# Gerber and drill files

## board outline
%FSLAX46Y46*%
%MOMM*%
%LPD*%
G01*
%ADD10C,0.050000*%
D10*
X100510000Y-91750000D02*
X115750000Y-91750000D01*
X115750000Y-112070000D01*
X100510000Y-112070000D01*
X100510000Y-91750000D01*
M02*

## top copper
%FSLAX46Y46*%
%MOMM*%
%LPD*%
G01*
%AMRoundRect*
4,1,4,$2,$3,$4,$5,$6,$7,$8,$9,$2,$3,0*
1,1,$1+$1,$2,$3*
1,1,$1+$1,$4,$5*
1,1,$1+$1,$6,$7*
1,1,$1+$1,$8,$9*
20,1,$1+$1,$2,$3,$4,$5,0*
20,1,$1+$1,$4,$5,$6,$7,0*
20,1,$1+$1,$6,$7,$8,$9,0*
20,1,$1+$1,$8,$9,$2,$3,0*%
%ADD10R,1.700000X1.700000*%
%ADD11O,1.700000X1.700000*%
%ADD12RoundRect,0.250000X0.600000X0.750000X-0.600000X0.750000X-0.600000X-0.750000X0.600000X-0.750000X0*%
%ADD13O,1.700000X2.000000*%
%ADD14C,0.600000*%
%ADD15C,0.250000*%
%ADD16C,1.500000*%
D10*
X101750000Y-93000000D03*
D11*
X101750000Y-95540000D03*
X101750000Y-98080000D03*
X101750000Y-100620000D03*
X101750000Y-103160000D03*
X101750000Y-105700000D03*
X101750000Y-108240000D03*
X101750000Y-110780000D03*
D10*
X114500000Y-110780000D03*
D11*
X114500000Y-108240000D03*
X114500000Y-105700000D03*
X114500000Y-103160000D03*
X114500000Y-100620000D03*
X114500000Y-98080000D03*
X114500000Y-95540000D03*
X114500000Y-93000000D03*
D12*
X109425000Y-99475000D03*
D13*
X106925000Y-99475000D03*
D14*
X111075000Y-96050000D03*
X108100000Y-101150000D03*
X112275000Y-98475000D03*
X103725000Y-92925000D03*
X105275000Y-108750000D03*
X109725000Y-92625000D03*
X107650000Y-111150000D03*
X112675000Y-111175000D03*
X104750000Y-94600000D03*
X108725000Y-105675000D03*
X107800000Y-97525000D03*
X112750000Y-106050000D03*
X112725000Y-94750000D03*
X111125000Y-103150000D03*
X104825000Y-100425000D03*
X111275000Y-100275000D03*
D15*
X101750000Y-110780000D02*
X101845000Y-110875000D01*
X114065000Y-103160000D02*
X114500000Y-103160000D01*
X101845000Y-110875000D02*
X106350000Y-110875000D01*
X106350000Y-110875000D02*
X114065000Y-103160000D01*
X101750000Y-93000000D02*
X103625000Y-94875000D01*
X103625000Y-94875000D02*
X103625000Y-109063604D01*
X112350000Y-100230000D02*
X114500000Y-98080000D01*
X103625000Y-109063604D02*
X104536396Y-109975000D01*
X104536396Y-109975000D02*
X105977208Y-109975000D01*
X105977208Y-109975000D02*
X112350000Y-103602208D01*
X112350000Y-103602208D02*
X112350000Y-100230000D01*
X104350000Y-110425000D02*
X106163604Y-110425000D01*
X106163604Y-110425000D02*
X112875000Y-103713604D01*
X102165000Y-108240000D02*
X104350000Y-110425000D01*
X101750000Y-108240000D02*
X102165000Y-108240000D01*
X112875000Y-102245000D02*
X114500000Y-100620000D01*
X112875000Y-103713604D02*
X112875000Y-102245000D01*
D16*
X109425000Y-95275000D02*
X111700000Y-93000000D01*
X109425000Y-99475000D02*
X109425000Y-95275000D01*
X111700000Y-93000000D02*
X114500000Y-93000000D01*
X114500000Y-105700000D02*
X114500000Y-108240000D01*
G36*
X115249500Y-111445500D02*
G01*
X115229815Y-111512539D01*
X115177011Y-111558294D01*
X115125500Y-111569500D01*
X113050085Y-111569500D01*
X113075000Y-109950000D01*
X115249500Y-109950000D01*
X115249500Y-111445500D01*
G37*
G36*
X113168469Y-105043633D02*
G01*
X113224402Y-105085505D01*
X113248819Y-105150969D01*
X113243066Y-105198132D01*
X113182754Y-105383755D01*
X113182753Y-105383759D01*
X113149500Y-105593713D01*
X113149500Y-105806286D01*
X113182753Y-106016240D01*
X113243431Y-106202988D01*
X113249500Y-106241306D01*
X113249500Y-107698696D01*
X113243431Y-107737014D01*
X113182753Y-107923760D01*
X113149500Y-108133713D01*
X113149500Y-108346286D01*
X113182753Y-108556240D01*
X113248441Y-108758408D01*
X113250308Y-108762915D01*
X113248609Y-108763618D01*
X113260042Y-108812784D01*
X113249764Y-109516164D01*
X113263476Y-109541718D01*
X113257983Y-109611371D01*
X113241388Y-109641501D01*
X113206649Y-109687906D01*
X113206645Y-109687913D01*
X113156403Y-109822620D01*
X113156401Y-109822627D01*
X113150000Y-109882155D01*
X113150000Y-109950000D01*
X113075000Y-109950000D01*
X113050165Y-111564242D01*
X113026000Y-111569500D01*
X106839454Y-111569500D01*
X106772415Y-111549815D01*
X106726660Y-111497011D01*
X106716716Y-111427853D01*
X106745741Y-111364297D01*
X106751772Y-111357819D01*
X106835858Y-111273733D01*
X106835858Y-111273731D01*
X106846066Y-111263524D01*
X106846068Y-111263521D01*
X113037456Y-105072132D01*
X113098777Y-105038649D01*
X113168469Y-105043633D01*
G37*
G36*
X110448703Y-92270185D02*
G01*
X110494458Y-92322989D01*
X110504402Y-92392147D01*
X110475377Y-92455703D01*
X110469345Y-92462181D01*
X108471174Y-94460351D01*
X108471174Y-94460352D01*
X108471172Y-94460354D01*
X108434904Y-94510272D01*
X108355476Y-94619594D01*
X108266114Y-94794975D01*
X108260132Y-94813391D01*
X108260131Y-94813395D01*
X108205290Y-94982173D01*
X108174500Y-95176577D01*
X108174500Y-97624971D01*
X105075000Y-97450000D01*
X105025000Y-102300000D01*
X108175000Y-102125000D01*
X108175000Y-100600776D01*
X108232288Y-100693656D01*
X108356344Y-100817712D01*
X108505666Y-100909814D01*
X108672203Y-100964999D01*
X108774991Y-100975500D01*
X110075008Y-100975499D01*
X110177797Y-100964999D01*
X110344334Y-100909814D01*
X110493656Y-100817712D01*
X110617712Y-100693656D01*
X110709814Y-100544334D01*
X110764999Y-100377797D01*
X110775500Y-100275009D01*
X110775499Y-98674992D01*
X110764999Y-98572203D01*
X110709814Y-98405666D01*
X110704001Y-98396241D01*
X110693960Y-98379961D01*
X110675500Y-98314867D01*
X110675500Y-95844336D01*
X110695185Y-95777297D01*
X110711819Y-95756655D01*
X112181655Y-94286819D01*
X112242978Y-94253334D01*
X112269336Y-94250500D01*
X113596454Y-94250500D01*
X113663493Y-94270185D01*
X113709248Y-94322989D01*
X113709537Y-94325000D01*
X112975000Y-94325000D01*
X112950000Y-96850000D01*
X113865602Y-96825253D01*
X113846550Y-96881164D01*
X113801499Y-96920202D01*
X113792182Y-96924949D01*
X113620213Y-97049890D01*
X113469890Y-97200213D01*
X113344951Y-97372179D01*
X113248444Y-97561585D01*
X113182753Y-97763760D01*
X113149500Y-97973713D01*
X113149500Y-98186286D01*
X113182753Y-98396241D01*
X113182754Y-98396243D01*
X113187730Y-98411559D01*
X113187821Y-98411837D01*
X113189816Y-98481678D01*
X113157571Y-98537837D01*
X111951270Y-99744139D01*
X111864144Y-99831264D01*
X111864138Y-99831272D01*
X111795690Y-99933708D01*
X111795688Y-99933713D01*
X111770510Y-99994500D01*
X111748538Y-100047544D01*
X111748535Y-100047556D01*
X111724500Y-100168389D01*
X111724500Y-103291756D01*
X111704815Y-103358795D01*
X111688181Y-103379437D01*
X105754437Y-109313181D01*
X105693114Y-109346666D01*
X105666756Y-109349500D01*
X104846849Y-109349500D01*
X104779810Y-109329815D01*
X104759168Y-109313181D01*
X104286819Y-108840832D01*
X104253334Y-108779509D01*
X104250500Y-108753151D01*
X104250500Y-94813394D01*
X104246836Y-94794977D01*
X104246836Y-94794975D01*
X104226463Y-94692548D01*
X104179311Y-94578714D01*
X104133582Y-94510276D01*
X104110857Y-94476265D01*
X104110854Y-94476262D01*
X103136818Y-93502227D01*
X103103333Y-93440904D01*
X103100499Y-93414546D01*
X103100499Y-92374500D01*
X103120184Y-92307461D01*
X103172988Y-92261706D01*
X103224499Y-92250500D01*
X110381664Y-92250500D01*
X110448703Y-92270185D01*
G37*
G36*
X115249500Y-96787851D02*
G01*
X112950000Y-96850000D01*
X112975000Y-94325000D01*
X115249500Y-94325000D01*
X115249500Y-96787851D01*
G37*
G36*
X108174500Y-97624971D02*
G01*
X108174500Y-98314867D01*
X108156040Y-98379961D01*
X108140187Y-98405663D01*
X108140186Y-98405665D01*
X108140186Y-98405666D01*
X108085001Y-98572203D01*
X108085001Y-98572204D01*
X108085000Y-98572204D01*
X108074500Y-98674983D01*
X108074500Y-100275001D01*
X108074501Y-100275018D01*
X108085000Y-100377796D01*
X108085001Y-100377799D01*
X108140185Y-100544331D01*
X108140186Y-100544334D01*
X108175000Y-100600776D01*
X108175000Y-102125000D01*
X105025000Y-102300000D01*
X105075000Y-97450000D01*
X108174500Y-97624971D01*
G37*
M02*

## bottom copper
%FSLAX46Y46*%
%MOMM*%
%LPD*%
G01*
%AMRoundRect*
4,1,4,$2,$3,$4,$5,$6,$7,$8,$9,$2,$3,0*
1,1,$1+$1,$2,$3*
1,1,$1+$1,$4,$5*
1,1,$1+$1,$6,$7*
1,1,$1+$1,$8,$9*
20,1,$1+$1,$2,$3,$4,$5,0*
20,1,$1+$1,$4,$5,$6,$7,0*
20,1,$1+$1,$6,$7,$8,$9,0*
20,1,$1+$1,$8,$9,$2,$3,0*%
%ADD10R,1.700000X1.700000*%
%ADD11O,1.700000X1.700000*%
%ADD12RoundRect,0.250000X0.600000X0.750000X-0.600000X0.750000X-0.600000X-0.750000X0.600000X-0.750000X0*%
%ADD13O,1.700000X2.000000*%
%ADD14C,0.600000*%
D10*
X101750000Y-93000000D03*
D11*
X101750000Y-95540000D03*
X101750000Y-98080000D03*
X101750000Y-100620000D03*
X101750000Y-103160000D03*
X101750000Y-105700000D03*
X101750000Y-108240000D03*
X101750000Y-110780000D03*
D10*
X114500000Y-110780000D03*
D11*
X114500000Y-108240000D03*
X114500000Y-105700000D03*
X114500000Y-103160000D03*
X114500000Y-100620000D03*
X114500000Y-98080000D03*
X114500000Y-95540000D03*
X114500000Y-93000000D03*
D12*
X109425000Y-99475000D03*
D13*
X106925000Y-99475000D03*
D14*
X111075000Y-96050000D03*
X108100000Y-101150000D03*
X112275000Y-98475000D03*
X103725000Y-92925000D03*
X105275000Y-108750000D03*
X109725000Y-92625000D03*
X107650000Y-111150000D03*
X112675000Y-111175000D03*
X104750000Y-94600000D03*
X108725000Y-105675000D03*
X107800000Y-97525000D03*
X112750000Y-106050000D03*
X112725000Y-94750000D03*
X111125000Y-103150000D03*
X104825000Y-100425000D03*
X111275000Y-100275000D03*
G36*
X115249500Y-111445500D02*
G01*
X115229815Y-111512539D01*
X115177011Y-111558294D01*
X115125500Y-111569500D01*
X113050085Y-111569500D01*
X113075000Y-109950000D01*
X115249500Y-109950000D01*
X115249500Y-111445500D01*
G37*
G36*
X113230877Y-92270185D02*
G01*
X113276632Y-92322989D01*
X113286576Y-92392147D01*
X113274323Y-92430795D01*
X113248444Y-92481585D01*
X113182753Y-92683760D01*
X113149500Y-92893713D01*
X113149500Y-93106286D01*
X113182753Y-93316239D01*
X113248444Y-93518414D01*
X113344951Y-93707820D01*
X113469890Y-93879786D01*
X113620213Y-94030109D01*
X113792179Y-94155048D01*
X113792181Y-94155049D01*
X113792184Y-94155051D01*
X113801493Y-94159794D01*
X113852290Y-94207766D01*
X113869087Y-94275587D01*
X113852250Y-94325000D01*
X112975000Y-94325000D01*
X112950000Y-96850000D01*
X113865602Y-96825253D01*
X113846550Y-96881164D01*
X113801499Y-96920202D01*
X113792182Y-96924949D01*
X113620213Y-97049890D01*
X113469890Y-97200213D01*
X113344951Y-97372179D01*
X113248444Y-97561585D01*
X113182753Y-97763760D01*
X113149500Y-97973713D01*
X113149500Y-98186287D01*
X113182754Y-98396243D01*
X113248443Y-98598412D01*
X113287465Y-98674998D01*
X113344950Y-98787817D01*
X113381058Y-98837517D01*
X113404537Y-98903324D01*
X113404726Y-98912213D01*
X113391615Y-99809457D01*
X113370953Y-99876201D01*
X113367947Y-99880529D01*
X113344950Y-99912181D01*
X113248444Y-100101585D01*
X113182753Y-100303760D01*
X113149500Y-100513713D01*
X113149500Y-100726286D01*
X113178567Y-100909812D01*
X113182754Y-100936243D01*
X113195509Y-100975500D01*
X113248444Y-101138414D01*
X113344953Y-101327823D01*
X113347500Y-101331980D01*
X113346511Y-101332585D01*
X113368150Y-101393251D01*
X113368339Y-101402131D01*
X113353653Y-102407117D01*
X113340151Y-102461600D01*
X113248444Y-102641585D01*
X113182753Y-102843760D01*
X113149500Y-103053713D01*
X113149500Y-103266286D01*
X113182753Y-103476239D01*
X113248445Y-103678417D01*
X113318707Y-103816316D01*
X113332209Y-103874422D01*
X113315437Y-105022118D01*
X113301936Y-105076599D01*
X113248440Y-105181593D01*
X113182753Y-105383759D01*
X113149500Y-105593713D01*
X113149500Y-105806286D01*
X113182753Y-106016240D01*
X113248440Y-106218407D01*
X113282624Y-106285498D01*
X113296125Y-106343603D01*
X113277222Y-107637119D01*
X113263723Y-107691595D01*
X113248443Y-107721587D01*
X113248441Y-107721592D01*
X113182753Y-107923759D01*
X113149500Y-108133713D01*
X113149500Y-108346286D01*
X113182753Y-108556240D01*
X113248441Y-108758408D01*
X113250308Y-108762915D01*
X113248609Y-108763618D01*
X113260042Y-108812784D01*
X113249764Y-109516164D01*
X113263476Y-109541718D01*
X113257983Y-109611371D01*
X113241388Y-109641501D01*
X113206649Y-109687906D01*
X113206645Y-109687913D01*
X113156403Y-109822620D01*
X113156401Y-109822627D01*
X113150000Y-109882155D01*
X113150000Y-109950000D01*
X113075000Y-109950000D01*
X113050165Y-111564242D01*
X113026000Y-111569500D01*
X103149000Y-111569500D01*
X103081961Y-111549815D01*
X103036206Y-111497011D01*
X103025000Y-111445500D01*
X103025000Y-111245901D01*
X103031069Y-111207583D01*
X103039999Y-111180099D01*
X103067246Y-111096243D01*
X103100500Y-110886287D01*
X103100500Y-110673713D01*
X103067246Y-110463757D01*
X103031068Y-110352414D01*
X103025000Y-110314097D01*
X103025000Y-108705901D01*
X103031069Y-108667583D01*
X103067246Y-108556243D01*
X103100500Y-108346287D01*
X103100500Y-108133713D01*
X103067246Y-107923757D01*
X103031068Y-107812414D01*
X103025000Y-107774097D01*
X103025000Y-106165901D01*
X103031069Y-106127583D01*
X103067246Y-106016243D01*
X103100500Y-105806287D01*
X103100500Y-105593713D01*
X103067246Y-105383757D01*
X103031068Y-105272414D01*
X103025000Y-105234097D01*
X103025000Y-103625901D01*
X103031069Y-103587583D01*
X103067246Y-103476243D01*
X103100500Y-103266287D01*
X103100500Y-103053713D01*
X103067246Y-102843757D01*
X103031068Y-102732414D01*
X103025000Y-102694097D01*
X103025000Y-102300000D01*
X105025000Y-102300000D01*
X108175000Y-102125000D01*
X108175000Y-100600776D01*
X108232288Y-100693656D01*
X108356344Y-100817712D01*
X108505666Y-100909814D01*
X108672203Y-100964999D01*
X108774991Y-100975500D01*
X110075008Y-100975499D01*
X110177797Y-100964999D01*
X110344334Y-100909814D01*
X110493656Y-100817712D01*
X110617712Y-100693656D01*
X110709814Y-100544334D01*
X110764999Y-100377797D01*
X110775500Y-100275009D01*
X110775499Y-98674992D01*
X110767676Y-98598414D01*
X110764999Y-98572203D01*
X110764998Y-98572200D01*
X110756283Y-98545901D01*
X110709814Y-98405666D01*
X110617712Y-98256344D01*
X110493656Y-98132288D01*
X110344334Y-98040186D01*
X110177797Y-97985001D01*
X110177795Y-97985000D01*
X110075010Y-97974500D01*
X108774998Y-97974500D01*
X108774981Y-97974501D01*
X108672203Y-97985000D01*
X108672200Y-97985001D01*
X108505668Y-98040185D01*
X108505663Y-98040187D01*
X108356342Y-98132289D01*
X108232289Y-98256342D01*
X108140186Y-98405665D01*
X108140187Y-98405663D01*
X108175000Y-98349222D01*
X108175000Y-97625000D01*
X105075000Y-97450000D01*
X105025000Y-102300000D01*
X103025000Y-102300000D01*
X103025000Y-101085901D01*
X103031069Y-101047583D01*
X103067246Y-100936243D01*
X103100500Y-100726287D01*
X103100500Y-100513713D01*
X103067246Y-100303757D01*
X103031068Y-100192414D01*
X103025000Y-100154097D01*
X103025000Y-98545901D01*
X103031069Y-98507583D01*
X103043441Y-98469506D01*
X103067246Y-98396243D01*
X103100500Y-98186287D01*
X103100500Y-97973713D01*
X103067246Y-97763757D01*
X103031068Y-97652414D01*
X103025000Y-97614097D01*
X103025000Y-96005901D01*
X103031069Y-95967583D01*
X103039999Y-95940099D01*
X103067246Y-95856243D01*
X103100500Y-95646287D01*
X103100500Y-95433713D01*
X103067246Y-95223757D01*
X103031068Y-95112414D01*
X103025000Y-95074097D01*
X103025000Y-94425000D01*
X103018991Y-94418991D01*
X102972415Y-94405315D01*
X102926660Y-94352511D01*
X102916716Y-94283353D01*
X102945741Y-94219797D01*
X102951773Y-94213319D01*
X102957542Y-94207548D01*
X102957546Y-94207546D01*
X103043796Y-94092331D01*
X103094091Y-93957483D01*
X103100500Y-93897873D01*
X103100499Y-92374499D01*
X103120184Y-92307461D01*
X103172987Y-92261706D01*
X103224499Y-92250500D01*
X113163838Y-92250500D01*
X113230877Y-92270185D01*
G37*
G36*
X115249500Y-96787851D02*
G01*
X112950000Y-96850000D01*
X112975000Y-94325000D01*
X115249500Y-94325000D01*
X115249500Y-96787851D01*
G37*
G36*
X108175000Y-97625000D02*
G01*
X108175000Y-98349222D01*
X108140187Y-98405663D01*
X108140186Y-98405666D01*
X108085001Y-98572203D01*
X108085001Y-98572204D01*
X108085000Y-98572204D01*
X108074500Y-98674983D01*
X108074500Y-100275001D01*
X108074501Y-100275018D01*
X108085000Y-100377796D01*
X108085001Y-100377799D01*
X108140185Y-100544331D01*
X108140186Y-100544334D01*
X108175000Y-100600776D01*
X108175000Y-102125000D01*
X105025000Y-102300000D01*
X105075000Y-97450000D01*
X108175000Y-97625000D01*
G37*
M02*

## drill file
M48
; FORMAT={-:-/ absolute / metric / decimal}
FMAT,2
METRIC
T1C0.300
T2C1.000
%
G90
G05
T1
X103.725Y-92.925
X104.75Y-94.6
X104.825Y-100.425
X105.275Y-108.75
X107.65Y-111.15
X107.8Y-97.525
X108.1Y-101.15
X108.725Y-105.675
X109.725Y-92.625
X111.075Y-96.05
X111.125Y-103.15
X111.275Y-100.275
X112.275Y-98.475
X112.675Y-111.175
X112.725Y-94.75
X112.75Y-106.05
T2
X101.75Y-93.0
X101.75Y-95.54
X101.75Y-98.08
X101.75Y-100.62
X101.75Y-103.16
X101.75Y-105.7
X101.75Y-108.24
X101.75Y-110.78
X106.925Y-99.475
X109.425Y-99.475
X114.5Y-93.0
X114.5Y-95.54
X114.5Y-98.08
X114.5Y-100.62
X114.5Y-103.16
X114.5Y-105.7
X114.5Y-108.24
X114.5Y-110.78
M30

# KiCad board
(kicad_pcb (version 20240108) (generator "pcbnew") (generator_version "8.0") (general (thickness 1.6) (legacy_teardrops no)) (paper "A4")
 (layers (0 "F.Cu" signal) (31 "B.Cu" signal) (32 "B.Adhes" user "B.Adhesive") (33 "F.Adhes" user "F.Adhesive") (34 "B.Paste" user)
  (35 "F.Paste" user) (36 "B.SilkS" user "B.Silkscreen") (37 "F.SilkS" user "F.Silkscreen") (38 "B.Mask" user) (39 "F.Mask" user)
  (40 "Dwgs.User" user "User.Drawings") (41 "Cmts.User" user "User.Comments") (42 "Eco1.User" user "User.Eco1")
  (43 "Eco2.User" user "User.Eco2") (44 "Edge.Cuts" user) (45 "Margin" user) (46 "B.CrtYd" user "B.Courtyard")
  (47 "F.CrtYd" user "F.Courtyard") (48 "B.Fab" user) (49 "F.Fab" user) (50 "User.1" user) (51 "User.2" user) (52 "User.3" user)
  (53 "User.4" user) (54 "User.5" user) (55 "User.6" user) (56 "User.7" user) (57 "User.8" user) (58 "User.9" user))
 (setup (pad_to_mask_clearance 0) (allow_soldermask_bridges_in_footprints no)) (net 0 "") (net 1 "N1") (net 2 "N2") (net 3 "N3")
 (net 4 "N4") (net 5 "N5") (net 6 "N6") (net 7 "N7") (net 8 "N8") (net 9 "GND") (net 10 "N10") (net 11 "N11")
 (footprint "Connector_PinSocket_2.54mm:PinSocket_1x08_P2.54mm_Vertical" (layer "F.Cu") (at 101.75 93)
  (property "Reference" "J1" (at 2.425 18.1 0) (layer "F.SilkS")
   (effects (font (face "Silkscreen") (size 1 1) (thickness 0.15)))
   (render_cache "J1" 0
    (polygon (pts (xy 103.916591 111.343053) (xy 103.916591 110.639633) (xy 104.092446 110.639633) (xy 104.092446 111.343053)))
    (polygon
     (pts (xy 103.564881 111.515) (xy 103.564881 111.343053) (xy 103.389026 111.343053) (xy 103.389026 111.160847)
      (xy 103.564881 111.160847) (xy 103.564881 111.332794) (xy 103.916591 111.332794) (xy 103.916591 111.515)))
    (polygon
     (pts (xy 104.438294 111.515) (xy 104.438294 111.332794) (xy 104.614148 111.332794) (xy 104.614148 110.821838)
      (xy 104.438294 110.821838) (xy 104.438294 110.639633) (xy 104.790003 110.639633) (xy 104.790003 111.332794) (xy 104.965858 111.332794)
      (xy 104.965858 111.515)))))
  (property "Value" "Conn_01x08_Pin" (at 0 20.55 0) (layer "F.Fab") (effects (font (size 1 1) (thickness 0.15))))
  (pad "1" thru_hole rect (at 0 0) (size 1.7 1.7) (drill 1) (layers "*.Cu" "*.Mask") (remove_unused_layers no) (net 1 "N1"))
  (pad "2" thru_hole oval (at 0 2.54) (size 1.7 1.7) (drill 1) (layers "*.Cu" "*.Mask") (remove_unused_layers no) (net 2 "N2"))
  (pad "3" thru_hole oval (at 0 5.08) (size 1.7 1.7) (drill 1) (layers "*.Cu" "*.Mask") (remove_unused_layers no) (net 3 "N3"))
  (pad "4" thru_hole oval (at 0 7.62) (size 1.7 1.7) (drill 1) (layers "*.Cu" "*.Mask") (remove_unused_layers no) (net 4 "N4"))
  (pad "5" thru_hole oval (at 0 10.16) (size 1.7 1.7) (drill 1) (layers "*.Cu" "*.Mask") (remove_unused_layers no) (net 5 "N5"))
  (pad "6" thru_hole oval (at 0 12.7) (size 1.7 1.7) (drill 1) (layers "*.Cu" "*.Mask") (remove_unused_layers no) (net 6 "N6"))
  (pad "7" thru_hole oval (at 0 15.24) (size 1.7 1.7) (drill 1) (layers "*.Cu" "*.Mask") (remove_unused_layers no) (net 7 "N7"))
  (pad "8" thru_hole oval (at 0 17.78) (size 1.7 1.7) (drill 1) (layers "*.Cu" "*.Mask") (remove_unused_layers no) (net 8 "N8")))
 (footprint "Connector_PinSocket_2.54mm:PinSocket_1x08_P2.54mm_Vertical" (layer "F.Cu") (at 114.5 110.78 180)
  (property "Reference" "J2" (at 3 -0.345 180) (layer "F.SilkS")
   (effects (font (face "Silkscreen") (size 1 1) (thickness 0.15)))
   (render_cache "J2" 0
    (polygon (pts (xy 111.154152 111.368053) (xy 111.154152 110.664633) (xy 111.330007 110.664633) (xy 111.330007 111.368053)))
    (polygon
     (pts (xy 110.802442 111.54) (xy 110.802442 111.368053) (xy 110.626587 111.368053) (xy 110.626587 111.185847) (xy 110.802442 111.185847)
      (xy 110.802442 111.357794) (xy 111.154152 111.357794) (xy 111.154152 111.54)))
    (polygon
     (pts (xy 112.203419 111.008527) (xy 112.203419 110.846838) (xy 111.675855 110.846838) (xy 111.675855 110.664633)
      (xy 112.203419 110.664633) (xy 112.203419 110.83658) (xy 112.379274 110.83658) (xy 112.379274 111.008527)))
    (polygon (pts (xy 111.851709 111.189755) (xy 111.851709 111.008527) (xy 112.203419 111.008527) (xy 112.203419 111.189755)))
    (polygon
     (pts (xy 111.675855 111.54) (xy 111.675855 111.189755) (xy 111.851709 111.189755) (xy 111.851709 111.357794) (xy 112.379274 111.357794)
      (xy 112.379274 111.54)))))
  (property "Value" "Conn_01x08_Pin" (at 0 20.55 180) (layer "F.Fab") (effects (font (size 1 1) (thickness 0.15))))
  (pad "1" thru_hole rect (at 0 0 180) (size 1.7 1.7) (drill 1) (layers "*.Cu" "*.Mask") (remove_unused_layers no) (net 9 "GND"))
  (pad "2" thru_hole oval (at 0 2.54 180) (size 1.7 1.7) (drill 1) (layers "*.Cu" "*.Mask") (remove_unused_layers no) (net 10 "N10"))
  (pad "3" thru_hole oval (at 0 5.08 180) (size 1.7 1.7) (drill 1) (layers "*.Cu" "*.Mask") (remove_unused_layers no) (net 10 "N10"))
  (pad "4" thru_hole oval (at 0 7.62 180) (size 1.7 1.7) (drill 1) (layers "*.Cu" "*.Mask") (remove_unused_layers no) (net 8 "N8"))
  (pad "5" thru_hole oval (at 0 10.16 180) (size 1.7 1.7) (drill 1) (layers "*.Cu" "*.Mask") (remove_unused_layers no) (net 7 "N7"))
  (pad "6" thru_hole oval (at 0 12.7 180) (size 1.7 1.7) (drill 1) (layers "*.Cu" "*.Mask") (remove_unused_layers no) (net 1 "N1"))
  (pad "7" thru_hole oval (at 0 15.24 180) (size 1.7 1.7) (drill 1) (layers "*.Cu" "*.Mask") (remove_unused_layers no) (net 9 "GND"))
  (pad "8" thru_hole oval (at 0 17.78 180) (size 1.7 1.7) (drill 1) (layers "*.Cu" "*.Mask") (remove_unused_layers no) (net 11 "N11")))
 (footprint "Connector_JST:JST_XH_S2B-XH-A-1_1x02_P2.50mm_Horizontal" (layer "F.Cu") (at 109.425 99.475 180)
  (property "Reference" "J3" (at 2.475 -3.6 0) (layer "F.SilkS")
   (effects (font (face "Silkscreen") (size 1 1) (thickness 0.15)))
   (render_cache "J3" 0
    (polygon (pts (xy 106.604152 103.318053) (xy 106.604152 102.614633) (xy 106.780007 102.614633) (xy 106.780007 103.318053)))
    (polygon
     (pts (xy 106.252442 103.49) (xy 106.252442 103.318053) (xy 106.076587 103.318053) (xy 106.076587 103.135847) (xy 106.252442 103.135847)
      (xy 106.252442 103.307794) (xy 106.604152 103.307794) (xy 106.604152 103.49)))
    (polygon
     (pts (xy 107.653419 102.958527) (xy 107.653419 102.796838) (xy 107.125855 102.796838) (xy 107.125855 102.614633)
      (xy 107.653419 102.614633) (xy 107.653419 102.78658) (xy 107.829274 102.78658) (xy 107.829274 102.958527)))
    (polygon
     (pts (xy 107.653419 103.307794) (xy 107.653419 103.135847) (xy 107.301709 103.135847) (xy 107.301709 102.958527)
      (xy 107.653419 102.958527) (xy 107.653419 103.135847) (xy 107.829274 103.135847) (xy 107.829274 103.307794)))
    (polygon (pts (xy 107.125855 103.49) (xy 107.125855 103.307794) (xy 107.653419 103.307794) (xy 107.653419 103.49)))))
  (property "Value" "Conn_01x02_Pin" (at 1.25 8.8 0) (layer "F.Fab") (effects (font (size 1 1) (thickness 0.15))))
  (pad "1" thru_hole roundrect (at 0 0 180) (size 1.7 2) (drill 1) (layers "*.Cu" "*.Mask") (remove_unused_layers no)
   (roundrect_rratio 0.147059) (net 11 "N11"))
  (pad "2" thru_hole oval (at 2.5 0 180) (size 1.7 2) (drill 1) (layers "*.Cu" "*.Mask") (remove_unused_layers no) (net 9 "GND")))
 (gr_rect (start 100.51 91.75) (end 115.75 112.07) (stroke (width 0.05) (type default)) (fill none) (layer "Edge.Cuts"))
 (segment (start 101.75 110.78) (end 101.845 110.875) (width 0.25) (layer "F.Cu") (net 8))
 (segment (start 114.065 103.16) (end 114.5 103.16) (width 0.25) (layer "F.Cu") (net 8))
 (segment (start 101.845 110.875) (end 106.35 110.875) (width 0.25) (layer "F.Cu") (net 8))
 (segment (start 106.35 110.875) (end 114.065 103.16) (width 0.25) (layer "F.Cu") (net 8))
 (segment (start 101.75 93) (end 103.625 94.875) (width 0.25) (layer "F.Cu") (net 1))
 (segment (start 103.625 94.875) (end 103.625 109.063604) (width 0.25) (layer "F.Cu") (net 1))
 (segment (start 112.35 100.23) (end 114.5 98.08) (width 0.25) (layer "F.Cu") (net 1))
 (segment (start 103.625 109.063604) (end 104.536396 109.975) (width 0.25) (layer "F.Cu") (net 1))
 (segment (start 104.536396 109.975) (end 105.977208 109.975) (width 0.25) (layer "F.Cu") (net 1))
 (segment (start 105.977208 109.975) (end 112.35 103.602208) (width 0.25) (layer "F.Cu") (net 1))
 (segment (start 112.35 103.602208) (end 112.35 100.23) (width 0.25) (layer "F.Cu") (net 1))
 (segment (start 104.35 110.425) (end 106.163604 110.425) (width 0.25) (layer "F.Cu") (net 7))
 (segment (start 106.163604 110.425) (end 112.875 103.713604) (width 0.25) (layer "F.Cu") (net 7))
 (segment (start 102.165 108.24) (end 104.35 110.425) (width 0.25) (layer "F.Cu") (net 7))
 (segment (start 101.75 108.24) (end 102.165 108.24) (width 0.25) (layer "F.Cu") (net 7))
 (segment (start 112.875 102.245) (end 114.5 100.62) (width 0.25) (layer "F.Cu") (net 7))
 (segment (start 112.875 103.713604) (end 112.875 102.245) (width 0.25) (layer "F.Cu") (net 7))
 (segment (start 109.425 95.275) (end 111.7 93) (width 1.5) (layer "F.Cu") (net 11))
 (segment (start 109.425 99.475) (end 109.425 95.275) (width 1.5) (layer "F.Cu") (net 11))
 (segment (start 111.7 93) (end 114.5 93) (width 1.5) (layer "F.Cu") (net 11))
 (via (at 111.075 96.05) (size 0.6) (drill 0.3) (layers "F.Cu" "B.Cu") (free yes) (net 9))
 (via (at 108.1 101.15) (size 0.6) (drill 0.3) (layers "F.Cu" "B.Cu") (free yes) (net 9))
 (via (at 112.275 98.475) (size 0.6) (drill 0.3) (layers "F.Cu" "B.Cu") (free yes) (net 9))
 (via (at 103.725 92.925) (size 0.6) (drill 0.3) (layers "F.Cu" "B.Cu") (free yes) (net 9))
 (via (at 105.275 108.75) (size 0.6) (drill 0.3) (layers "F.Cu" "B.Cu") (free yes) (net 9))
 (via (at 109.725 92.625) (size 0.6) (drill 0.3) (layers "F.Cu" "B.Cu") (free yes) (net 9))
 (via (at 107.65 111.15) (size 0.6) (drill 0.3) (layers "F.Cu" "B.Cu") (free yes) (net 9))
 (via (at 112.675 111.175) (size 0.6) (drill 0.3) (layers "F.Cu" "B.Cu") (free yes) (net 9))
 (via (at 104.75 94.6) (size 0.6) (drill 0.3) (layers "F.Cu" "B.Cu") (free yes) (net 9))
 (via (at 108.725 105.675) (size 0.6) (drill 0.3) (layers "F.Cu" "B.Cu") (free yes) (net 9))
 (via (at 107.8 97.525) (size 0.6) (drill 0.3) (layers "F.Cu" "B.Cu") (free yes) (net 9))
 (via (at 112.75 106.05) (size 0.6) (drill 0.3) (layers "F.Cu" "B.Cu") (free yes) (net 9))
 (via (at 112.725 94.75) (size 0.6) (drill 0.3) (layers "F.Cu" "B.Cu") (free yes) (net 9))
 (via (at 111.125 103.15) (size 0.6) (drill 0.3) (layers "F.Cu" "B.Cu") (free yes) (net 9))
 (via (at 104.825 100.425) (size 0.6) (drill 0.3) (layers "F.Cu" "B.Cu") (free yes) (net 9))
 (via (at 111.275 100.275) (size 0.6) (drill 0.3) (layers "F.Cu" "B.Cu") (free yes) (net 9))
 (segment (start 114.5 105.7) (end 114.5 108.24) (width 1.5) (layer "F.Cu") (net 10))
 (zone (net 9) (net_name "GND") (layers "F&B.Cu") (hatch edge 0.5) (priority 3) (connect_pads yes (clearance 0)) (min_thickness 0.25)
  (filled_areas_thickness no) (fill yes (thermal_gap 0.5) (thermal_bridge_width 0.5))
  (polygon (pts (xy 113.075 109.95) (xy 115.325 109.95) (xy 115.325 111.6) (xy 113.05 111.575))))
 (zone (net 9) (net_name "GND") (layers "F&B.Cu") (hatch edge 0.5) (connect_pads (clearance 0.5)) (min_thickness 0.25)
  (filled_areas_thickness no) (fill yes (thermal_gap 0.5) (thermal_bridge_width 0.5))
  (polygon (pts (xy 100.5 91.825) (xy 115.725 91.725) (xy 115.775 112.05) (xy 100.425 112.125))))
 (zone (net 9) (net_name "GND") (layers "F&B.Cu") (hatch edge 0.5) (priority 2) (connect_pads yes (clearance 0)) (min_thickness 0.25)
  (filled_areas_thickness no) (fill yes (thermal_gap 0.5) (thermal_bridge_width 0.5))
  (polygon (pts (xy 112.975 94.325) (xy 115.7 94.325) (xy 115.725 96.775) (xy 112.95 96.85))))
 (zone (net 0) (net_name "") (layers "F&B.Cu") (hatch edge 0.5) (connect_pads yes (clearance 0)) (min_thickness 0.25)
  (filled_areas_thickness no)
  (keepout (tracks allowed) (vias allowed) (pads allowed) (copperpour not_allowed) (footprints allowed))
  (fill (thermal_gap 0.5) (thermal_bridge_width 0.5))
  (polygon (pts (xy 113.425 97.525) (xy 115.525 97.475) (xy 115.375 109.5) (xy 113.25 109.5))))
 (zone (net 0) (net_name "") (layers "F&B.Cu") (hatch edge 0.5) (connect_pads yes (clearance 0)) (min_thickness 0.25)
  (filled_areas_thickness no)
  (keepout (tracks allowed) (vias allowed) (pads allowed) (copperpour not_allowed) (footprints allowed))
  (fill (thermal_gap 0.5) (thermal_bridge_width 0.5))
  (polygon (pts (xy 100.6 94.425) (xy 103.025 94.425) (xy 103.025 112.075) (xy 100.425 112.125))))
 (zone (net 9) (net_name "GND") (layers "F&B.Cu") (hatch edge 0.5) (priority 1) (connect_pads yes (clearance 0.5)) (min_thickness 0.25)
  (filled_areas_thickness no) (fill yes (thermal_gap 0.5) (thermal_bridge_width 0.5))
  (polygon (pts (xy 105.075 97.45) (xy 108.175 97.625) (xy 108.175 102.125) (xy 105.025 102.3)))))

